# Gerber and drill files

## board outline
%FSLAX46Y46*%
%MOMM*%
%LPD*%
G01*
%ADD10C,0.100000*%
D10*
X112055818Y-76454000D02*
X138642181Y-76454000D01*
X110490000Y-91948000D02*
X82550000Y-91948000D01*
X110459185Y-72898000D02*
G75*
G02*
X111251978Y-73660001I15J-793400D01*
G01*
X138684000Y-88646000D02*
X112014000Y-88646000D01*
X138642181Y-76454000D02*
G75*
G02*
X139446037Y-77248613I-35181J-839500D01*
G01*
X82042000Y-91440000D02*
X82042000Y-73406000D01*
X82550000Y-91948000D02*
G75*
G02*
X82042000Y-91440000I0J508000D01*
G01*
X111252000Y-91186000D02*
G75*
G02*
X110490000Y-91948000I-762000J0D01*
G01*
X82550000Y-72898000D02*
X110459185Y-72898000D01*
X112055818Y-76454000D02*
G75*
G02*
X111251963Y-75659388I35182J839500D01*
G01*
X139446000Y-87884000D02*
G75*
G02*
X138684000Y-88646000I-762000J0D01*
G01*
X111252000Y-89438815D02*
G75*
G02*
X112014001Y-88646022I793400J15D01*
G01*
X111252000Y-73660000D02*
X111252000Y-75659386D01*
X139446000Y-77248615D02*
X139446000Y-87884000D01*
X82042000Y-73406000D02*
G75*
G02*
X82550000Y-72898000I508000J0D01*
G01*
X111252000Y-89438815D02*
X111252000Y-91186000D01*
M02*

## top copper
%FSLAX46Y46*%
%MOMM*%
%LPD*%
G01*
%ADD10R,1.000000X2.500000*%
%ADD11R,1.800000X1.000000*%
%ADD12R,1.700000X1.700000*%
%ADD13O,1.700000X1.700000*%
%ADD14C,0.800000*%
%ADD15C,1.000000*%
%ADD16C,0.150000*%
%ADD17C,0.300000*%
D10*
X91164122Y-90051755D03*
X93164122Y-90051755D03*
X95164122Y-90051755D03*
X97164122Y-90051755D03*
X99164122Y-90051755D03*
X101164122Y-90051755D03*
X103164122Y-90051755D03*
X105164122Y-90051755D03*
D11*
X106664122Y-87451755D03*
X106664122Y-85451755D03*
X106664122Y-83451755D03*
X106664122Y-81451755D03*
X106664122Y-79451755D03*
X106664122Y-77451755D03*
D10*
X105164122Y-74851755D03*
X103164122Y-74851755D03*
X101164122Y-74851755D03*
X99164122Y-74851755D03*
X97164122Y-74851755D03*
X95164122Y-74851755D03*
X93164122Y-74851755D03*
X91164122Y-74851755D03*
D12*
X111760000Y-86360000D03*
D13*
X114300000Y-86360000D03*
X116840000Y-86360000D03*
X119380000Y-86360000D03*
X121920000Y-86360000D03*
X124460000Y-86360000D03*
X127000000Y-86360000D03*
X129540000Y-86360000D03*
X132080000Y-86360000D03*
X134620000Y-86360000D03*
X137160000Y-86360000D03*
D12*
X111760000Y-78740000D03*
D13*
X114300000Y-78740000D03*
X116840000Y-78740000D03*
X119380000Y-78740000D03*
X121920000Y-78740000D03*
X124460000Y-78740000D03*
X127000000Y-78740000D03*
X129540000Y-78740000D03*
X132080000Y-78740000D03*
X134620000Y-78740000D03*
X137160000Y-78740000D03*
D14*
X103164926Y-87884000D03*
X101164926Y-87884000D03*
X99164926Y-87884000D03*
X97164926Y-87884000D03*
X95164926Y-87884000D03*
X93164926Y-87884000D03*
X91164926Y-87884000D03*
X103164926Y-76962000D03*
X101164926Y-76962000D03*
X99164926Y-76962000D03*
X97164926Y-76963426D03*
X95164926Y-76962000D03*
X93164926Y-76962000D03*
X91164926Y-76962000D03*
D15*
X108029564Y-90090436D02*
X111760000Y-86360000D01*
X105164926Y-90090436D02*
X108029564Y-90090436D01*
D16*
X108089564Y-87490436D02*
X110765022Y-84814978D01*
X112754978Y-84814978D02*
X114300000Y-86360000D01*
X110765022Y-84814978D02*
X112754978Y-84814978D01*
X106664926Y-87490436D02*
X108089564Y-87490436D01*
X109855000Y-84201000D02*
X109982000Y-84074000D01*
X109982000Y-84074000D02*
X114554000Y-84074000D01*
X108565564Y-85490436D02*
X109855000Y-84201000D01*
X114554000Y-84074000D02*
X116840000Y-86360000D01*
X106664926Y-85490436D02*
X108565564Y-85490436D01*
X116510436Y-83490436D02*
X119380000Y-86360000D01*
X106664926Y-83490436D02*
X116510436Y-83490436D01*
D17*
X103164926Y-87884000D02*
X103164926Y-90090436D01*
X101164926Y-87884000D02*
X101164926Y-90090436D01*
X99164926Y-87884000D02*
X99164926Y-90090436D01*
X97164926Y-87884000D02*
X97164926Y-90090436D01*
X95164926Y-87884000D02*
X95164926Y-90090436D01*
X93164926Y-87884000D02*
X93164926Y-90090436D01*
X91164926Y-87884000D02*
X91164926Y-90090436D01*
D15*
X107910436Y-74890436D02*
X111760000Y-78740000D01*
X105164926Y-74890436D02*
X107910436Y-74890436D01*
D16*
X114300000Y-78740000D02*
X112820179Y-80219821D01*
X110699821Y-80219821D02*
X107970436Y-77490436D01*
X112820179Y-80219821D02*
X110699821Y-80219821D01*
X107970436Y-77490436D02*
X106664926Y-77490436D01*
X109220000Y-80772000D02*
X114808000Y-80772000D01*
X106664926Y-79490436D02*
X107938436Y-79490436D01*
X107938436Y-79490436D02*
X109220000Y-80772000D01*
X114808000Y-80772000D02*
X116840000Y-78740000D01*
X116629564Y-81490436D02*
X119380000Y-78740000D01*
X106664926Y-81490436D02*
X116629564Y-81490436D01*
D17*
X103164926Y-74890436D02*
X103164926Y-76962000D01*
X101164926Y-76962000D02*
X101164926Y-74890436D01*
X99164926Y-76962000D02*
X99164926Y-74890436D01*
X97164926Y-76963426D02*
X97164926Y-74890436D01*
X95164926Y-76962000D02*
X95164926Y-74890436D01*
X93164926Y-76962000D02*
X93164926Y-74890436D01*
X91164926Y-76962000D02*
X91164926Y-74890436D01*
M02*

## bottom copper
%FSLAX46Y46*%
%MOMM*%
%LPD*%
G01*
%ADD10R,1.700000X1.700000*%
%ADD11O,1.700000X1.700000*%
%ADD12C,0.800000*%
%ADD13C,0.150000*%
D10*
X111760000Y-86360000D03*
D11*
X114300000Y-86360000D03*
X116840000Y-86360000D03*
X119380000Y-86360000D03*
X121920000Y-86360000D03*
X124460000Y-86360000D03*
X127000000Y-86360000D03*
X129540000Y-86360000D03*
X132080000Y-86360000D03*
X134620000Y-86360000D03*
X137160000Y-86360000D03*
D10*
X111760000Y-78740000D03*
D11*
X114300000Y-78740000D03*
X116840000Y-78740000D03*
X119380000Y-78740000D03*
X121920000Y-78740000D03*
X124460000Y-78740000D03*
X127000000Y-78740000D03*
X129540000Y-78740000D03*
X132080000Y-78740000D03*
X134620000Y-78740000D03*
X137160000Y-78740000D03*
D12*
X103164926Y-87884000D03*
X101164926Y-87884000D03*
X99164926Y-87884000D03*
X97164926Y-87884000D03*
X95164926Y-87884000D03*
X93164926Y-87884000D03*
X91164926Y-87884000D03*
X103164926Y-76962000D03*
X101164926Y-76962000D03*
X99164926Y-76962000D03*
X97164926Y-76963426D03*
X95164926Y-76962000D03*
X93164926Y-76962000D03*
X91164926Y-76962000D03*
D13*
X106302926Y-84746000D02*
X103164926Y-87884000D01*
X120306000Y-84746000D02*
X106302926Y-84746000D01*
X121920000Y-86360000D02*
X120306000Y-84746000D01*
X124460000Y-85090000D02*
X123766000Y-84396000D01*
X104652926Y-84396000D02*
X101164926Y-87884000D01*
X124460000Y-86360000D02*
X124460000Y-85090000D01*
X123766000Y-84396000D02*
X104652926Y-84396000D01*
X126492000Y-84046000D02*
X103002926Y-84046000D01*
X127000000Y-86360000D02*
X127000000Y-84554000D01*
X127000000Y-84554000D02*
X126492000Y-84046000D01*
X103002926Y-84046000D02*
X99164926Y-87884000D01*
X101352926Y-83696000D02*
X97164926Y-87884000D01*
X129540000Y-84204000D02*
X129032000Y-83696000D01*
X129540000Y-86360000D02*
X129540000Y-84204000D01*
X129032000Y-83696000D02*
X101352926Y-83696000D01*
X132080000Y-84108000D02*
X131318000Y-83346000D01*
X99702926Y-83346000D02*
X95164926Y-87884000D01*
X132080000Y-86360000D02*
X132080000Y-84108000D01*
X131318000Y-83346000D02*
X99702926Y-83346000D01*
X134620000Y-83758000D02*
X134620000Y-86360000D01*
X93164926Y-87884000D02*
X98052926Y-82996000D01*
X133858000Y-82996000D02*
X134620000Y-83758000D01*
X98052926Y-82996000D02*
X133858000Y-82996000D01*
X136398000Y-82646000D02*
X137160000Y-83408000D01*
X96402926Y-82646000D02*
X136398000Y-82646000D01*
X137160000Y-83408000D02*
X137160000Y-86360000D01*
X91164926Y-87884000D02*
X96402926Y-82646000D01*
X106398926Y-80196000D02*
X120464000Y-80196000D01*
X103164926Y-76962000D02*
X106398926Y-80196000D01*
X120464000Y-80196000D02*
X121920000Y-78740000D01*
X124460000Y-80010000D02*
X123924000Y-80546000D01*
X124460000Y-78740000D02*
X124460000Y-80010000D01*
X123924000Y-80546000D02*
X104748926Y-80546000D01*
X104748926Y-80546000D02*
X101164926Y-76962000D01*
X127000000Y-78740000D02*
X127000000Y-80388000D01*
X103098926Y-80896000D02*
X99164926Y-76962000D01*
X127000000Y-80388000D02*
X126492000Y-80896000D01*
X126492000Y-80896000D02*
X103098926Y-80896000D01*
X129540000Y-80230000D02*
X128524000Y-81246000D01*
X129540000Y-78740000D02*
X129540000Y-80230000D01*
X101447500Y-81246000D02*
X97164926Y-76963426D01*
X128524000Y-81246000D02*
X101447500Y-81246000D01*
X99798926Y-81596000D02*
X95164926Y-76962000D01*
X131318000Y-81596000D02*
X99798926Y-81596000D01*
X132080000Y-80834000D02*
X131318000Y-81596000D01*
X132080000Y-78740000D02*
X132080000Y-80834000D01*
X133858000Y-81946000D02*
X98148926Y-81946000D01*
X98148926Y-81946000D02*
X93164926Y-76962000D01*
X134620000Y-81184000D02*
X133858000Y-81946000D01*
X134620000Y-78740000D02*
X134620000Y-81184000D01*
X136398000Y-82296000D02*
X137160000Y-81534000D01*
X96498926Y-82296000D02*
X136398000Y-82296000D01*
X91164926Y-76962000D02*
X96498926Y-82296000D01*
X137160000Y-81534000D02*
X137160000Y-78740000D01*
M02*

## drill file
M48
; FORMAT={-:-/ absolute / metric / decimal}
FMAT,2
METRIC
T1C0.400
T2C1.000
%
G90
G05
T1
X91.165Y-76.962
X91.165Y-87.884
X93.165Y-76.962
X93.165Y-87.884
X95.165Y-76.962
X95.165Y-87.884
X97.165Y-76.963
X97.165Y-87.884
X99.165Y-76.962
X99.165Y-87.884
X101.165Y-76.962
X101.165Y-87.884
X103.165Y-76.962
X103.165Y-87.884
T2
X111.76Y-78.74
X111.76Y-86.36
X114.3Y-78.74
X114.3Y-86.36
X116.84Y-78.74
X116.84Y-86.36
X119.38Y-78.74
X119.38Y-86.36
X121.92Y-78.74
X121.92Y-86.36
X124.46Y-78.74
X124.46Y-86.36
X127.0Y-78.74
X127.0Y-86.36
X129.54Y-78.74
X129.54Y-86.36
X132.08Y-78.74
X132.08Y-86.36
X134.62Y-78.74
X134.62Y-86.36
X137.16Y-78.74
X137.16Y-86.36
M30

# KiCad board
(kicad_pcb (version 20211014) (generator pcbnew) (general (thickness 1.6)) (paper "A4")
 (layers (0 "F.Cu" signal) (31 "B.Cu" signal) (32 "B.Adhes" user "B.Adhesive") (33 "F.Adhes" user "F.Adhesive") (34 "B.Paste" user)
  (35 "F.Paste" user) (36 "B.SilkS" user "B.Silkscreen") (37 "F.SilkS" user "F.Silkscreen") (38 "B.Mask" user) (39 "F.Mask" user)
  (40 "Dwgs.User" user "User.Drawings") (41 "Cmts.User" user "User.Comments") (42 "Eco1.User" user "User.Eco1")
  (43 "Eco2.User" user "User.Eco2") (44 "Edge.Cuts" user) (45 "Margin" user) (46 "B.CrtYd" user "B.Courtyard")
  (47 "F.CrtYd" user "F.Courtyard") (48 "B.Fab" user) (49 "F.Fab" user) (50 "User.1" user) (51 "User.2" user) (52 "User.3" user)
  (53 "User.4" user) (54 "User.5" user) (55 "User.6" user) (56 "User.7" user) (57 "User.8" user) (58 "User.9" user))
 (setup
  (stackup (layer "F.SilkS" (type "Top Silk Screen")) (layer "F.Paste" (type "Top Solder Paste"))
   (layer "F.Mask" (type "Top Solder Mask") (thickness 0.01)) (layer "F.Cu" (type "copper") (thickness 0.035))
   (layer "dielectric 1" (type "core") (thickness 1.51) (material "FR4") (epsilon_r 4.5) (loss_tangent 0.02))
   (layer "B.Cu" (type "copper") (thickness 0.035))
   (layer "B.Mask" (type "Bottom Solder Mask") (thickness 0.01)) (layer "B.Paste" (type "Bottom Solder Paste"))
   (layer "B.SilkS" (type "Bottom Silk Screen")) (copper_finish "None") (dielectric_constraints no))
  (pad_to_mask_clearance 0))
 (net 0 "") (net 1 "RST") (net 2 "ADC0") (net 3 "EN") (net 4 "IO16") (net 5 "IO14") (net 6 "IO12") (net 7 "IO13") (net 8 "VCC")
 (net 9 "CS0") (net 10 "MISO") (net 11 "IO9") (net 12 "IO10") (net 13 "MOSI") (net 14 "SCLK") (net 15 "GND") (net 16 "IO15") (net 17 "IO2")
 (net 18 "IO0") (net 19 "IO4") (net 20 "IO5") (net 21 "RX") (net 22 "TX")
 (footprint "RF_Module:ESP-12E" (layer "F.Cu") (at 94.664122 82.451755 90)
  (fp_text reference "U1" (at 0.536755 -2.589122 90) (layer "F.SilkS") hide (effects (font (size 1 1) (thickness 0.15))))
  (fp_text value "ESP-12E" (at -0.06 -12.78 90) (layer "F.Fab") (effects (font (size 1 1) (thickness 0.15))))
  (pad "1" smd rect (at -7.6 -3.5 90) (size 2.5 1) (layers "F.Cu" "F.Paste" "F.Mask") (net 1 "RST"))
  (pad "2" smd rect (at -7.6 -1.5 90) (size 2.5 1) (layers "F.Cu" "F.Paste" "F.Mask") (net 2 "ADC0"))
  (pad "3" smd rect (at -7.6 0.5 90) (size 2.5 1) (layers "F.Cu" "F.Paste" "F.Mask") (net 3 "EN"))
  (pad "4" smd rect (at -7.6 2.5 90) (size 2.5 1) (layers "F.Cu" "F.Paste" "F.Mask") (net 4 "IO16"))
  (pad "5" smd rect (at -7.6 4.5 90) (size 2.5 1) (layers "F.Cu" "F.Paste" "F.Mask") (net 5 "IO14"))
  (pad "6" smd rect (at -7.6 6.5 90) (size 2.5 1) (layers "F.Cu" "F.Paste" "F.Mask") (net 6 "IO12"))
  (pad "7" smd rect (at -7.6 8.5 90) (size 2.5 1) (layers "F.Cu" "F.Paste" "F.Mask") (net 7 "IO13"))
  (pad "8" smd rect (at -7.6 10.5 90) (size 2.5 1) (layers "F.Cu" "F.Paste" "F.Mask") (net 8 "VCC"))
  (pad "9" smd rect (at -5 12 90) (size 1 1.8) (layers "F.Cu" "F.Paste" "F.Mask") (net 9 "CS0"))
  (pad "10" smd rect (at -3 12 90) (size 1 1.8) (layers "F.Cu" "F.Paste" "F.Mask") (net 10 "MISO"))
  (pad "11" smd rect (at -1 12 90) (size 1 1.8) (layers "F.Cu" "F.Paste" "F.Mask") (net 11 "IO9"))
  (pad "12" smd rect (at 1 12 90) (size 1 1.8) (layers "F.Cu" "F.Paste" "F.Mask") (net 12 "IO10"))
  (pad "13" smd rect (at 3 12 90) (size 1 1.8) (layers "F.Cu" "F.Paste" "F.Mask") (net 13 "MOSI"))
  (pad "14" smd rect (at 5 12 90) (size 1 1.8) (layers "F.Cu" "F.Paste" "F.Mask") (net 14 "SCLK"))
  (pad "15" smd rect (at 7.6 10.5 90) (size 2.5 1) (layers "F.Cu" "F.Paste" "F.Mask") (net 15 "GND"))
  (pad "16" smd rect (at 7.6 8.5 90) (size 2.5 1) (layers "F.Cu" "F.Paste" "F.Mask") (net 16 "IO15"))
  (pad "17" smd rect (at 7.6 6.5 90) (size 2.5 1) (layers "F.Cu" "F.Paste" "F.Mask") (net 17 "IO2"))
  (pad "18" smd rect (at 7.6 4.5 90) (size 2.5 1) (layers "F.Cu" "F.Paste" "F.Mask") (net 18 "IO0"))
  (pad "19" smd rect (at 7.6 2.5 90) (size 2.5 1) (layers "F.Cu" "F.Paste" "F.Mask") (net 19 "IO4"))
  (pad "20" smd rect (at 7.6 0.5 90) (size 2.5 1) (layers "F.Cu" "F.Paste" "F.Mask") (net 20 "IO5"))
  (pad "21" smd rect (at 7.6 -1.5 90) (size 2.5 1) (layers "F.Cu" "F.Paste" "F.Mask") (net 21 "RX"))
  (pad "22" smd rect (at 7.6 -3.5 90) (size 2.5 1) (layers "F.Cu" "F.Paste" "F.Mask") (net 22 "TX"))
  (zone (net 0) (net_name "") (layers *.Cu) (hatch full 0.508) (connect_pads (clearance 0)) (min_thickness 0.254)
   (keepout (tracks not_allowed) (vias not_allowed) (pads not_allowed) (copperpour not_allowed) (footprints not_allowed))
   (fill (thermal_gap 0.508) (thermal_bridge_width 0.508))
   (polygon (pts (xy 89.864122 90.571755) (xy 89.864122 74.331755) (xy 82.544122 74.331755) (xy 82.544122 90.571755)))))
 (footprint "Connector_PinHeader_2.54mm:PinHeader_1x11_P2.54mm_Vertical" (layer "B.Cu") (at 111.76 86.36 -90)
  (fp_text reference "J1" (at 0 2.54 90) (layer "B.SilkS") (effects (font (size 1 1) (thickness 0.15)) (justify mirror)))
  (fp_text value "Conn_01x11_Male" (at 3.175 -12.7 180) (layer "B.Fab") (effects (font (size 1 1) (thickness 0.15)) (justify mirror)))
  (pad "1" thru_hole rect (at 0 0 270) (size 1.7 1.7) (drill 1) (layers *.Cu *.Mask) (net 8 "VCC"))
  (pad "2" thru_hole oval (at 0 -2.54 270) (size 1.7 1.7) (drill 1) (layers *.Cu *.Mask) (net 9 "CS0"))
  (pad "3" thru_hole oval (at 0 -5.08 270) (size 1.7 1.7) (drill 1) (layers *.Cu *.Mask) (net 10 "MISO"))
  (pad "4" thru_hole oval (at 0 -7.62 270) (size 1.7 1.7) (drill 1) (layers *.Cu *.Mask) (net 11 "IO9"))
  (pad "5" thru_hole oval (at 0 -10.16 270) (size 1.7 1.7) (drill 1) (layers *.Cu *.Mask) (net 7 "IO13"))
  (pad "6" thru_hole oval (at 0 -12.7 270) (size 1.7 1.7) (drill 1) (layers *.Cu *.Mask) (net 6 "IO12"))
  (pad "7" thru_hole oval (at 0 -15.24 270) (size 1.7 1.7) (drill 1) (layers *.Cu *.Mask) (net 5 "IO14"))
  (pad "8" thru_hole oval (at 0 -17.78 270) (size 1.7 1.7) (drill 1) (layers *.Cu *.Mask) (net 4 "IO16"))
  (pad "9" thru_hole oval (at 0 -20.32 270) (size 1.7 1.7) (drill 1) (layers *.Cu *.Mask) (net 3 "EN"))
  (pad "10" thru_hole oval (at 0 -22.86 270) (size 1.7 1.7) (drill 1) (layers *.Cu *.Mask) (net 2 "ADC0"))
  (pad "11" thru_hole oval (at 0 -25.4 270) (size 1.7 1.7) (drill 1) (layers *.Cu *.Mask) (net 1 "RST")))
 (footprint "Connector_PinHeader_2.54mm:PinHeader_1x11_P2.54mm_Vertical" (layer "B.Cu") (at 111.76 78.74 -90)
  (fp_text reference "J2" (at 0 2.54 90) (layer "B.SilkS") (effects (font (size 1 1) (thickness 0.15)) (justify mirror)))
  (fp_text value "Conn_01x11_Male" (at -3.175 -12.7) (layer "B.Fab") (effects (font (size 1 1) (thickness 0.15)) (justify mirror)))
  (pad "1" thru_hole rect (at 0 0 270) (size 1.7 1.7) (drill 1) (layers *.Cu *.Mask) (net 15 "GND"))
  (pad "2" thru_hole oval (at 0 -2.54 270) (size 1.7 1.7) (drill 1) (layers *.Cu *.Mask) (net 14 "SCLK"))
  (pad "3" thru_hole oval (at 0 -5.08 270) (size 1.7 1.7) (drill 1) (layers *.Cu *.Mask) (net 13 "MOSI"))
  (pad "4" thru_hole oval (at 0 -7.62 270) (size 1.7 1.7) (drill 1) (layers *.Cu *.Mask) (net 12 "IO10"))
  (pad "5" thru_hole oval (at 0 -10.16 270) (size 1.7 1.7) (drill 1) (layers *.Cu *.Mask) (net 16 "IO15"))
  (pad "6" thru_hole oval (at 0 -12.7 270) (size 1.7 1.7) (drill 1) (layers *.Cu *.Mask) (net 17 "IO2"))
  (pad "7" thru_hole oval (at 0 -15.24 270) (size 1.7 1.7) (drill 1) (layers *.Cu *.Mask) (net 18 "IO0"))
  (pad "8" thru_hole oval (at 0 -17.78 270) (size 1.7 1.7) (drill 1) (layers *.Cu *.Mask) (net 19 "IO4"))
  (pad "9" thru_hole oval (at 0 -20.32 270) (size 1.7 1.7) (drill 1) (layers *.Cu *.Mask) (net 20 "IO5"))
  (pad "10" thru_hole oval (at 0 -22.86 270) (size 1.7 1.7) (drill 1) (layers *.Cu *.Mask) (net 21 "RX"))
  (pad "11" thru_hole oval (at 0 -25.4 270) (size 1.7 1.7) (drill 1) (layers *.Cu *.Mask) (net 22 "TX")))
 (gr_line (start 112.055818 76.454) (end 138.642181 76.454) (layer "Edge.Cuts") (width 0.1))
 (gr_line (start 110.49 91.948) (end 82.55 91.948) (layer "Edge.Cuts") (width 0.1))
 (gr_arc (start 110.459185 72.898) (mid 111.009003 73.119386) (end 111.252 73.66) (layer "Edge.Cuts") (width 0.1))
 (gr_line (start 138.684 88.646) (end 112.014 88.646) (layer "Edge.Cuts") (width 0.1))
 (gr_arc (start 138.642181 76.454) (mid 139.197678 76.695941) (end 139.446 77.248615) (layer "Edge.Cuts") (width 0.1))
 (gr_line (start 82.042 91.44) (end 82.042 73.406) (layer "Edge.Cuts") (width 0.1))
 (gr_arc (start 82.55 91.948) (mid 82.19079 91.79921) (end 82.042 91.44) (layer "Edge.Cuts") (width 0.1))
 (gr_arc (start 111.252 91.186) (mid 111.028815 91.724815) (end 110.49 91.948) (layer "Edge.Cuts") (width 0.1))
 (gr_line (start 82.55 72.898) (end 110.459185 72.898) (layer "Edge.Cuts") (width 0.1))
 (gr_arc (start 112.055818 76.454) (mid 111.500321 76.21206) (end 111.252 75.659386) (layer "Edge.Cuts") (width 0.1))
 (gr_arc (start 139.446 87.884) (mid 139.222815 88.422815) (end 138.684 88.646) (layer "Edge.Cuts") (width 0.1))
 (gr_arc (start 111.252 89.438815) (mid 111.473386 88.888997) (end 112.014 88.646) (layer "Edge.Cuts") (width 0.1))
 (gr_line (start 111.252 73.66) (end 111.252 75.659386) (layer "Edge.Cuts") (width 0.1))
 (gr_line (start 139.446 77.248615) (end 139.446 87.884) (layer "Edge.Cuts") (width 0.1))
 (gr_arc (start 82.042 73.406) (mid 82.19079 73.04679) (end 82.55 72.898) (layer "Edge.Cuts") (width 0.1))
 (gr_line (start 111.252 89.438815) (end 111.252 91.186) (layer "Edge.Cuts") (width 0.1))
 (segment (start 108.029564 90.090436) (end 111.76 86.36) (width 1) (layer "F.Cu") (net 8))
 (segment (start 105.164926 90.090436) (end 108.029564 90.090436) (width 1) (layer "F.Cu") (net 8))
 (segment (start 108.089564 87.490436) (end 110.765022 84.814978) (width 0.15) (layer "F.Cu") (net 9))
 (segment (start 112.754978 84.814978) (end 114.3 86.36) (width 0.15) (layer "F.Cu") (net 9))
 (segment (start 110.765022 84.814978) (end 112.754978 84.814978) (width 0.15) (layer "F.Cu") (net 9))
 (segment (start 106.664926 87.490436) (end 108.089564 87.490436) (width 0.15) (layer "F.Cu") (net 9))
 (segment (start 109.855 84.201) (end 109.982 84.074) (width 0.15) (layer "F.Cu") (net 10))
 (segment (start 109.982 84.074) (end 114.554 84.074) (width 0.15) (layer "F.Cu") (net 10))
 (segment (start 108.565564 85.490436) (end 109.855 84.201) (width 0.15) (layer "F.Cu") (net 10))
 (segment (start 114.554 84.074) (end 116.84 86.36) (width 0.15) (layer "F.Cu") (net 10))
 (segment (start 106.664926 85.490436) (end 108.565564 85.490436) (width 0.15) (layer "F.Cu") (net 10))
 (segment (start 116.510436 83.490436) (end 119.38 86.36) (width 0.15) (layer "F.Cu") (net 11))
 (segment (start 106.664926 83.490436) (end 116.510436 83.490436) (width 0.15) (layer "F.Cu") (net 11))
 (segment (start 103.164926 87.884) (end 103.164926 90.090436) (width 0.3) (layer "F.Cu") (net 7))
 (via (at 103.164926 87.884) (size 0.8) (drill 0.4) (layers "F.Cu" "B.Cu") (free) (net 7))
 (segment (start 106.302926 84.746) (end 103.164926 87.884) (width 0.15) (layer "B.Cu") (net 7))
 (segment (start 120.306 84.746) (end 106.302926 84.746) (width 0.15) (layer "B.Cu") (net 7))
 (segment (start 121.92 86.36) (end 120.306 84.746) (width 0.15) (layer "B.Cu") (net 7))
 (segment (start 101.164926 87.884) (end 101.164926 90.090436) (width 0.3) (layer "F.Cu") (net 6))
 (via (at 101.164926 87.884) (size 0.8) (drill 0.4) (layers "F.Cu" "B.Cu") (free) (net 6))
 (segment (start 124.46 85.09) (end 123.766 84.396) (width 0.15) (layer "B.Cu") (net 6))
 (segment (start 104.652926 84.396) (end 101.164926 87.884) (width 0.15) (layer "B.Cu") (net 6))
 (segment (start 124.46 86.36) (end 124.46 85.09) (width 0.15) (layer "B.Cu") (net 6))
 (segment (start 123.766 84.396) (end 104.652926 84.396) (width 0.15) (layer "B.Cu") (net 6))
 (segment (start 99.164926 87.884) (end 99.164926 90.090436) (width 0.3) (layer "F.Cu") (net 5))
 (via (at 99.164926 87.884) (size 0.8) (drill 0.4) (layers "F.Cu" "B.Cu") (free) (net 5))
 (segment (start 126.492 84.046) (end 103.002926 84.046) (width 0.15) (layer "B.Cu") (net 5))
 (segment (start 127 86.36) (end 127 84.554) (width 0.15) (layer "B.Cu") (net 5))
 (segment (start 127 84.554) (end 126.492 84.046) (width 0.15) (layer "B.Cu") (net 5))
 (segment (start 103.002926 84.046) (end 99.164926 87.884) (width 0.15) (layer "B.Cu") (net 5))
 (segment (start 97.164926 87.884) (end 97.164926 90.090436) (width 0.3) (layer "F.Cu") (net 4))
 (via (at 97.164926 87.884) (size 0.8) (drill 0.4) (layers "F.Cu" "B.Cu") (free) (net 4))
 (segment (start 101.352926 83.696) (end 97.164926 87.884) (width 0.15) (layer "B.Cu") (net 4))
 (segment (start 129.54 84.204) (end 129.032 83.696) (width 0.15) (layer "B.Cu") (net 4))
 (segment (start 129.54 86.36) (end 129.54 84.204) (width 0.15) (layer "B.Cu") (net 4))
 (segment (start 129.032 83.696) (end 101.352926 83.696) (width 0.15) (layer "B.Cu") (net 4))
 (segment (start 95.164926 87.884) (end 95.164926 90.090436) (width 0.3) (layer "F.Cu") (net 3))
 (via (at 95.164926 87.884) (size 0.8) (drill 0.4) (layers "F.Cu" "B.Cu") (free) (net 3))
 (segment (start 132.08 84.108) (end 131.318 83.346) (width 0.15) (layer "B.Cu") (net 3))
 (segment (start 99.702926 83.346) (end 95.164926 87.884) (width 0.15) (layer "B.Cu") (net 3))
 (segment (start 132.08 86.36) (end 132.08 84.108) (width 0.15) (layer "B.Cu") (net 3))
 (segment (start 131.318 83.346) (end 99.702926 83.346) (width 0.15) (layer "B.Cu") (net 3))
 (segment (start 93.164926 87.884) (end 93.164926 90.090436) (width 0.3) (layer "F.Cu") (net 2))
 (via (at 93.164926 87.884) (size 0.8) (drill 0.4) (layers "F.Cu" "B.Cu") (free) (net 2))
 (segment (start 134.62 83.758) (end 134.62 86.36) (width 0.15) (layer "B.Cu") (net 2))
 (segment (start 93.164926 87.884) (end 98.052926 82.996) (width 0.15) (layer "B.Cu") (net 2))
 (segment (start 133.858 82.996) (end 134.62 83.758) (width 0.15) (layer "B.Cu") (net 2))
 (segment (start 98.052926 82.996) (end 133.858 82.996) (width 0.15) (layer "B.Cu") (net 2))
 (segment (start 91.164926 87.884) (end 91.164926 90.090436) (width 0.3) (layer "F.Cu") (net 1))
 (via (at 91.164926 87.884) (size 0.8) (drill 0.4) (layers "F.Cu" "B.Cu") (free) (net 1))
 (segment (start 136.398 82.646) (end 137.16 83.408) (width 0.15) (layer "B.Cu") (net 1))
 (segment (start 96.402926 82.646) (end 136.398 82.646) (width 0.15) (layer "B.Cu") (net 1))
 (segment (start 137.16 83.408) (end 137.16 86.36) (width 0.15) (layer "B.Cu") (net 1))
 (segment (start 91.164926 87.884) (end 96.402926 82.646) (width 0.15) (layer "B.Cu") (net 1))
 (segment (start 107.910436 74.890436) (end 111.76 78.74) (width 1) (layer "F.Cu") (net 15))
 (segment (start 105.164926 74.890436) (end 107.910436 74.890436) (width 1) (layer "F.Cu") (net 15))
 (segment (start 114.3 78.74) (end 112.820179 80.219821) (width 0.15) (layer "F.Cu") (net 14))
 (segment (start 110.699821 80.219821) (end 107.970436 77.490436) (width 0.15) (layer "F.Cu") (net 14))
 (segment (start 112.820179 80.219821) (end 110.699821 80.219821) (width 0.15) (layer "F.Cu") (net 14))
 (segment (start 107.970436 77.490436) (end 106.664926 77.490436) (width 0.15) (layer "F.Cu") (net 14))
 (segment (start 109.22 80.772) (end 114.808 80.772) (width 0.15) (layer "F.Cu") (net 13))
 (segment (start 106.664926 79.490436) (end 107.938436 79.490436) (width 0.15) (layer "F.Cu") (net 13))
 (segment (start 107.938436 79.490436) (end 109.22 80.772) (width 0.15) (layer "F.Cu") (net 13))
 (segment (start 114.808 80.772) (end 116.84 78.74) (width 0.15) (layer "F.Cu") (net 13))
 (segment (start 116.629564 81.490436) (end 119.38 78.74) (width 0.15) (layer "F.Cu") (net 12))
 (segment (start 106.664926 81.490436) (end 116.629564 81.490436) (width 0.15) (layer "F.Cu") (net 12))
 (segment (start 103.164926 74.890436) (end 103.164926 76.962) (width 0.3) (layer "F.Cu") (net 16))
 (via (at 103.164926 76.962) (size 0.8) (drill 0.4) (layers "F.Cu" "B.Cu") (free) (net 16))
 (segment (start 106.398926 80.196) (end 120.464 80.196) (width 0.15) (layer "B.Cu") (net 16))
 (segment (start 103.164926 76.962) (end 106.398926 80.196) (width 0.15) (layer "B.Cu") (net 16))
 (segment (start 120.464 80.196) (end 121.92 78.74) (width 0.15) (layer "B.Cu") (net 16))
 (segment (start 101.164926 76.962) (end 101.164926 74.890436) (width 0.3) (layer "F.Cu") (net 17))
 (via (at 101.164926 76.962) (size 0.8) (drill 0.4) (layers "F.Cu" "B.Cu") (free) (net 17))
 (segment (start 124.46 80.01) (end 123.924 80.546) (width 0.15) (layer "B.Cu") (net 17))
 (segment (start 124.46 78.74) (end 124.46 80.01) (width 0.15) (layer "B.Cu") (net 17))
 (segment (start 123.924 80.546) (end 104.748926 80.546) (width 0.15) (layer "B.Cu") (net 17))
 (segment (start 104.748926 80.546) (end 101.164926 76.962) (width 0.15) (layer "B.Cu") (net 17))
 (segment (start 99.164926 76.962) (end 99.164926 74.890436) (width 0.3) (layer "F.Cu") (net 18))
 (via (at 99.164926 76.962) (size 0.8) (drill 0.4) (layers "F.Cu" "B.Cu") (free) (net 18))
 (segment (start 127 78.74) (end 127 80.388) (width 0.15) (layer "B.Cu") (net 18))
 (segment (start 103.098926 80.896) (end 99.164926 76.962) (width 0.15) (layer "B.Cu") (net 18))
 (segment (start 127 80.388) (end 126.492 80.896) (width 0.15) (layer "B.Cu") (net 18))
 (segment (start 126.492 80.896) (end 103.098926 80.896) (width 0.15) (layer "B.Cu") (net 18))
 (segment (start 97.164926 76.963426) (end 97.164926 74.890436) (width 0.3) (layer "F.Cu") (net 19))
 (via (at 97.164926 76.963426) (size 0.8) (drill 0.4) (layers "F.Cu" "B.Cu") (free) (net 19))
 (segment (start 129.54 80.23) (end 128.524 81.246) (width 0.15) (layer "B.Cu") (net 19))
 (segment (start 129.54 78.74) (end 129.54 80.23) (width 0.15) (layer "B.Cu") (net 19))
 (segment (start 101.4475 81.246) (end 97.164926 76.963426) (width 0.15) (layer "B.Cu") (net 19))
 (segment (start 128.524 81.246) (end 101.4475 81.246) (width 0.15) (layer "B.Cu") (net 19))
 (segment (start 95.164926 76.962) (end 95.164926 74.890436) (width 0.3) (layer "F.Cu") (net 20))
 (via (at 95.164926 76.962) (size 0.8) (drill 0.4) (layers "F.Cu" "B.Cu") (free) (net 20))
 (segment (start 99.798926 81.596) (end 95.164926 76.962) (width 0.15) (layer "B.Cu") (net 20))
 (segment (start 131.318 81.596) (end 99.798926 81.596) (width 0.15) (layer "B.Cu") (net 20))
 (segment (start 132.08 80.834) (end 131.318 81.596) (width 0.15) (layer "B.Cu") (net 20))
 (segment (start 132.08 78.74) (end 132.08 80.834) (width 0.15) (layer "B.Cu") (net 20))
 (segment (start 93.164926 76.962) (end 93.164926 74.890436) (width 0.3) (layer "F.Cu") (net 21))
 (via (at 93.164926 76.962) (size 0.8) (drill 0.4) (layers "F.Cu" "B.Cu") (free) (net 21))
 (segment (start 133.858 81.946) (end 98.148926 81.946) (width 0.15) (layer "B.Cu") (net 21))
 (segment (start 98.148926 81.946) (end 93.164926 76.962) (width 0.15) (layer "B.Cu") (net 21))
 (segment (start 134.62 81.184) (end 133.858 81.946) (width 0.15) (layer "B.Cu") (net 21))
 (segment (start 134.62 78.74) (end 134.62 81.184) (width 0.15) (layer "B.Cu") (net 21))
 (segment (start 91.164926 76.962) (end 91.164926 74.890436) (width 0.3) (layer "F.Cu") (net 22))
 (via (at 91.164926 76.962) (size 0.8) (drill 0.4) (layers "F.Cu" "B.Cu") (free) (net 22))
 (segment (start 136.398 82.296) (end 137.16 81.534) (width 0.15) (layer "B.Cu") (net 22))
 (segment (start 96.498926 82.296) (end 136.398 82.296) (width 0.15) (layer "B.Cu") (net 22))
 (segment (start 91.164926 76.962) (end 96.498926 82.296) (width 0.15) (layer "B.Cu") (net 22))
 (segment (start 137.16 81.534) (end 137.16 78.74) (width 0.15) (layer "B.Cu") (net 22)))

